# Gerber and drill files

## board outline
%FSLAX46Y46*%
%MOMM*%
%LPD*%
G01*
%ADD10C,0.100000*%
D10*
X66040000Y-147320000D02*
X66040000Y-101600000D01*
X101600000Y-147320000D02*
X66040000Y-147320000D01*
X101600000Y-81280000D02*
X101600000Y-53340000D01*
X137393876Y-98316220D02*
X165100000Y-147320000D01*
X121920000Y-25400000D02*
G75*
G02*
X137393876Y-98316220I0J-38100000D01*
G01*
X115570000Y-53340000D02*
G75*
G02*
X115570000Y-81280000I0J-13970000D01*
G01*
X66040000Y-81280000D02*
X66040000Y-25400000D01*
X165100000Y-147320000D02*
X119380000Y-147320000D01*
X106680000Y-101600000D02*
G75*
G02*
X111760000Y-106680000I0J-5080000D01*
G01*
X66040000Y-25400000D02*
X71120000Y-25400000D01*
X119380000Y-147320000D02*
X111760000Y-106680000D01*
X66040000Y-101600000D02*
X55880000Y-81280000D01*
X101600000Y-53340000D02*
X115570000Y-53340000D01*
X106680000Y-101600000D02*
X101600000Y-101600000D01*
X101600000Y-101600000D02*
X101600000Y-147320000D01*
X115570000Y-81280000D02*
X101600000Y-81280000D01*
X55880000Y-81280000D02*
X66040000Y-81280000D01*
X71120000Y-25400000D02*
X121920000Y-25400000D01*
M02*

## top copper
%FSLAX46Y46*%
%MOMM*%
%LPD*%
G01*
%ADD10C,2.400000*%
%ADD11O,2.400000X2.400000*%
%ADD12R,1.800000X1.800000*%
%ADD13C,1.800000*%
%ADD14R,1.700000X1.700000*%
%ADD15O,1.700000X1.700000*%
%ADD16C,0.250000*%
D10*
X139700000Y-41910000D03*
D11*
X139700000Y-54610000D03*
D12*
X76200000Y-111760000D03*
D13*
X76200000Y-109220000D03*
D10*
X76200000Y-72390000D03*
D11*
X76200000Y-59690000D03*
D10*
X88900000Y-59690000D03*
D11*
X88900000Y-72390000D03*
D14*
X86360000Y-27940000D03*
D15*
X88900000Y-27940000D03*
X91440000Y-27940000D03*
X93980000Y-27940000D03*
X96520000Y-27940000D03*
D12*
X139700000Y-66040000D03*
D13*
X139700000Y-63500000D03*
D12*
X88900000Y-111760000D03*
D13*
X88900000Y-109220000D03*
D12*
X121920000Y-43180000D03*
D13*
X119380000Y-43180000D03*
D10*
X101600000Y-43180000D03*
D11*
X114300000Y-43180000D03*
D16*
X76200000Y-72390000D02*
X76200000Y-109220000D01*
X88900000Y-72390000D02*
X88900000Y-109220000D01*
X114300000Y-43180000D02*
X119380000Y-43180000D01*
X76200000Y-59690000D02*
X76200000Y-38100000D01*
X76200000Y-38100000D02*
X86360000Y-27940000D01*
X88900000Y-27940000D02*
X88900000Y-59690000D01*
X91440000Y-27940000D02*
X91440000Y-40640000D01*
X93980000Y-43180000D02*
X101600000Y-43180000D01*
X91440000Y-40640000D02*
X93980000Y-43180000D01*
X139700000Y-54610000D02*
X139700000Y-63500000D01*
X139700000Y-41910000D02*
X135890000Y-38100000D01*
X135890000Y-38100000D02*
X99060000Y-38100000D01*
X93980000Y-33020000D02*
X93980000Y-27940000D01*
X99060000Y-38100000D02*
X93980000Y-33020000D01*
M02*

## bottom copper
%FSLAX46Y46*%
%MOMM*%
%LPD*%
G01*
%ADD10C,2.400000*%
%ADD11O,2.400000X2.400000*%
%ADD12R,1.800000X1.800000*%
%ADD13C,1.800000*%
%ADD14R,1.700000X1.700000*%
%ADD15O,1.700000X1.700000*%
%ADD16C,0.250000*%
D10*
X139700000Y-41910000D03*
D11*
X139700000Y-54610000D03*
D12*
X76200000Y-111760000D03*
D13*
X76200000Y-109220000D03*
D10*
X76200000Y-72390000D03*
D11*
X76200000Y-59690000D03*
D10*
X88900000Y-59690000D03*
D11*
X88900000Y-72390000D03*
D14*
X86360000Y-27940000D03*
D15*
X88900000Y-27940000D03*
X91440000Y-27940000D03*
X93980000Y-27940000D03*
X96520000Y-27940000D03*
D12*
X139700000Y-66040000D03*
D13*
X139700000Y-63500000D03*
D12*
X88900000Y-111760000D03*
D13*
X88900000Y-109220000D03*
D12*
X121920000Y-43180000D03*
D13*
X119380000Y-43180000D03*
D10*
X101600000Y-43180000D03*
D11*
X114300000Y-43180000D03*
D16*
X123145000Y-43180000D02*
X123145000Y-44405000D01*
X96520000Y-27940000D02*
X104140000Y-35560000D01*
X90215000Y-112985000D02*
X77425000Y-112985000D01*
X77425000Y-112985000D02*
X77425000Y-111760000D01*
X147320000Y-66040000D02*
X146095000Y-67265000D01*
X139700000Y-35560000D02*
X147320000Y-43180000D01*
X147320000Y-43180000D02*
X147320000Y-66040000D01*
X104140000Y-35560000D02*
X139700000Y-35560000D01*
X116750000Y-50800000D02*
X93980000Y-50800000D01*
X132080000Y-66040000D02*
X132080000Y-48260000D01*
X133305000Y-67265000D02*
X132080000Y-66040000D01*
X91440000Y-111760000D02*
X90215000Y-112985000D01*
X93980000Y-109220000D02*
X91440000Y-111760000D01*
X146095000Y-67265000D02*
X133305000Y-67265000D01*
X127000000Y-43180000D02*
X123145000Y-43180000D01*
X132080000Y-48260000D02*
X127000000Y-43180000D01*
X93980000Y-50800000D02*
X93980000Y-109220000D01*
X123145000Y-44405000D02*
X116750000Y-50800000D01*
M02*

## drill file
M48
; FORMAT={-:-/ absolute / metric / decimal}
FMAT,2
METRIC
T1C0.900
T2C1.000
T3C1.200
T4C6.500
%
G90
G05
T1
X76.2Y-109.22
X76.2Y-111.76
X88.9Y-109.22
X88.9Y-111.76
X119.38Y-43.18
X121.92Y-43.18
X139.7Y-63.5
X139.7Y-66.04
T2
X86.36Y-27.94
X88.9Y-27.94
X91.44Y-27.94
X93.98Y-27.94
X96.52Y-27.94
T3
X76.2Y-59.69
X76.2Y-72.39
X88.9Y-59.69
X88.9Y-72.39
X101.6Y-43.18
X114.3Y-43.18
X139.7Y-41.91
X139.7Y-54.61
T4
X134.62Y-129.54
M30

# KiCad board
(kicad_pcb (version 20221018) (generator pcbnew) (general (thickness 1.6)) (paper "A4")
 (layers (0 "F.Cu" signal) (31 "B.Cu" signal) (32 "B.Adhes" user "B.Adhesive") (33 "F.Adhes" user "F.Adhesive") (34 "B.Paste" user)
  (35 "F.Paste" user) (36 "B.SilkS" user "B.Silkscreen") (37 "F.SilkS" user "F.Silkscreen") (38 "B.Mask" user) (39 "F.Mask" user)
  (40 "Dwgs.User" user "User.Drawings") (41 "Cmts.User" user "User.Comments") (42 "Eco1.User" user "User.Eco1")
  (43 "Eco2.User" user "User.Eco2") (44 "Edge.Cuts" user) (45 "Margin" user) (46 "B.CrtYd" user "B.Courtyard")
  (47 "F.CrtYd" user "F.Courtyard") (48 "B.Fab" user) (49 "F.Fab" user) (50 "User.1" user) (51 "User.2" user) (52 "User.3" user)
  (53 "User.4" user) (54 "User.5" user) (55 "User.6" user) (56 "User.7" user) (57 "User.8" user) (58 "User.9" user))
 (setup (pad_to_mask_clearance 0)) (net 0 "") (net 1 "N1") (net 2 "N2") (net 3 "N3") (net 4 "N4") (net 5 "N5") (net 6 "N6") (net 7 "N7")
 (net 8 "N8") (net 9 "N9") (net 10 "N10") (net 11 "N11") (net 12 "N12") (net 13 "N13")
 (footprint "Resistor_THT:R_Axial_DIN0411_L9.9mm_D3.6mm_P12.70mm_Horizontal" (layer "F.Cu") (at 139.7 41.91 -90)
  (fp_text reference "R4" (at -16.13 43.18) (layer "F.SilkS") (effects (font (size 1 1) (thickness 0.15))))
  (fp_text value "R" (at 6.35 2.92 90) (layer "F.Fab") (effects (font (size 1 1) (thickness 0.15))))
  (pad "1" thru_hole circle (at 0 0 270) (size 2.4 2.4) (drill 1.2) (layers "*.Cu" "*.Mask") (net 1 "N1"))
  (pad "2" thru_hole oval (at 12.7 0 270) (size 2.4 2.4) (drill 1.2) (layers "*.Cu" "*.Mask") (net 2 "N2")))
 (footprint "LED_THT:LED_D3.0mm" (layer "F.Cu") (at 76.2 111.76 90)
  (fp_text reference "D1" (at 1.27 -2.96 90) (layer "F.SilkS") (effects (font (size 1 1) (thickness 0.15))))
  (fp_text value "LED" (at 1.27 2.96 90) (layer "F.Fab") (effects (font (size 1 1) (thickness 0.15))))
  (pad "1" thru_hole rect (at 0 0 90) (size 1.8 1.8) (drill 0.9) (layers "*.Cu" "*.Mask") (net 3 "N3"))
  (pad "2" thru_hole circle (at 2.54 0 90) (size 1.8 1.8) (drill 0.9) (layers "*.Cu" "*.Mask") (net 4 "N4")))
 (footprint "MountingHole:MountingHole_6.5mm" (layer "F.Cu") (at 134.62 129.54)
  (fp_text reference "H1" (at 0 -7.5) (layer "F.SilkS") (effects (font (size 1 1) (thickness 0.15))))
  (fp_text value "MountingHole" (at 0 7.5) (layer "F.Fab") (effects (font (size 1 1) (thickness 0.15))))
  (pad "" np_thru_hole circle (at 0 0) (size 6.5 6.5) (drill 6.5) (layers "*.Cu" "*.Mask")))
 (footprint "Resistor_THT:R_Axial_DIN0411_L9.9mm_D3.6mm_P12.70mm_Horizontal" (layer "F.Cu") (at 76.2 72.39 90)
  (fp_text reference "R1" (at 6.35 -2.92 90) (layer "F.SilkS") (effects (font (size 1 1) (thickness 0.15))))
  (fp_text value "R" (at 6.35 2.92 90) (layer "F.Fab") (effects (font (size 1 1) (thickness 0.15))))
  (pad "1" thru_hole circle (at 0 0 90) (size 2.4 2.4) (drill 1.2) (layers "*.Cu" "*.Mask") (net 4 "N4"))
  (pad "2" thru_hole oval (at 12.7 0 90) (size 2.4 2.4) (drill 1.2) (layers "*.Cu" "*.Mask") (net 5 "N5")))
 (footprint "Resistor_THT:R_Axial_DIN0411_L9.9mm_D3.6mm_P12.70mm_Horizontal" (layer "F.Cu") (at 88.9 59.69 -90)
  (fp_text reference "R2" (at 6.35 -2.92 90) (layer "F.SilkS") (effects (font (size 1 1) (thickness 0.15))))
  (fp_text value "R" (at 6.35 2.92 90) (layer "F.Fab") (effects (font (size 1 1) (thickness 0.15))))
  (pad "1" thru_hole circle (at 0 0 270) (size 2.4 2.4) (drill 1.2) (layers "*.Cu" "*.Mask") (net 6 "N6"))
  (pad "2" thru_hole oval (at 12.7 0 270) (size 2.4 2.4) (drill 1.2) (layers "*.Cu" "*.Mask") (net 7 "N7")))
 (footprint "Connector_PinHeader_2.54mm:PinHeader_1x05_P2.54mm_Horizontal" (layer "F.Cu") (at 86.36 27.94 90)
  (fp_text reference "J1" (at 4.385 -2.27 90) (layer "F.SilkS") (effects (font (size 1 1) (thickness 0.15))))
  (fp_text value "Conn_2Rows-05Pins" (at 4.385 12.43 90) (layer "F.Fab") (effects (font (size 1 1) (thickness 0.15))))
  (pad "1" thru_hole rect (at 0 0 90) (size 1.7 1.7) (drill 1) (layers "*.Cu" "*.Mask") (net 5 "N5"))
  (pad "2" thru_hole oval (at 0 2.54 90) (size 1.7 1.7) (drill 1) (layers "*.Cu" "*.Mask") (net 6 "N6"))
  (pad "3" thru_hole oval (at 0 5.08 90) (size 1.7 1.7) (drill 1) (layers "*.Cu" "*.Mask") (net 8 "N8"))
  (pad "4" thru_hole oval (at 0 7.62 90) (size 1.7 1.7) (drill 1) (layers "*.Cu" "*.Mask") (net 1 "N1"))
  (pad "5" thru_hole oval (at 0 10.16 90) (size 1.7 1.7) (drill 1) (layers "*.Cu" "*.Mask") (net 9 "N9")))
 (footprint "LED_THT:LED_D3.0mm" (layer "F.Cu") (at 139.7 66.04 90)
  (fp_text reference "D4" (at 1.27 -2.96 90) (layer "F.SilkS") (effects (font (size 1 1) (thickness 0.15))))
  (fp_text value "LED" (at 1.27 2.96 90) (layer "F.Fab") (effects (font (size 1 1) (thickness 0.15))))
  (pad "1" thru_hole rect (at 0 0 90) (size 1.8 1.8) (drill 0.9) (layers "*.Cu" "*.Mask") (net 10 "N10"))
  (pad "2" thru_hole circle (at 2.54 0 90) (size 1.8 1.8) (drill 0.9) (layers "*.Cu" "*.Mask") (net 2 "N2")))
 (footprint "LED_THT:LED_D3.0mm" (layer "F.Cu") (at 88.9 111.76 90)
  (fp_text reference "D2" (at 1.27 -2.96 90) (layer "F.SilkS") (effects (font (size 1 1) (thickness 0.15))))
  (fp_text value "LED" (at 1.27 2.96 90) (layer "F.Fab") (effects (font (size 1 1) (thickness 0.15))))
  (pad "1" thru_hole rect (at 0 0 90) (size 1.8 1.8) (drill 0.9) (layers "*.Cu" "*.Mask") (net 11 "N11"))
  (pad "2" thru_hole circle (at 2.54 0 90) (size 1.8 1.8) (drill 0.9) (layers "*.Cu" "*.Mask") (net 7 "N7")))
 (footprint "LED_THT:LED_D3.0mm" (layer "F.Cu") (at 121.92 43.18 180)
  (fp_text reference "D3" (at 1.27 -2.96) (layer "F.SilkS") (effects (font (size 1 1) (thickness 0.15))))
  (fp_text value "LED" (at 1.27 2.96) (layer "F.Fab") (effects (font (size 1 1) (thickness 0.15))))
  (pad "1" thru_hole rect (at 0 0 180) (size 1.8 1.8) (drill 0.9) (layers "*.Cu" "*.Mask") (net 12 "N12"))
  (pad "2" thru_hole circle (at 2.54 0 180) (size 1.8 1.8) (drill 0.9) (layers "*.Cu" "*.Mask") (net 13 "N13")))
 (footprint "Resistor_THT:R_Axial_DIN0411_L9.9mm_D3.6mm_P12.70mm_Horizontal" (layer "F.Cu") (at 101.6 43.18)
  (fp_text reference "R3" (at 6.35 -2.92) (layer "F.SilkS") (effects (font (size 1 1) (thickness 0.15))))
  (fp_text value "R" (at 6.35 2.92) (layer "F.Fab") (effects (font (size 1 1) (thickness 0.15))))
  (pad "1" thru_hole circle (at 0 0) (size 2.4 2.4) (drill 1.2) (layers "*.Cu" "*.Mask") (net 8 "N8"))
  (pad "2" thru_hole oval (at 12.7 0) (size 2.4 2.4) (drill 1.2) (layers "*.Cu" "*.Mask") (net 13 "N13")))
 (gr_line (start 66.04 147.32) (end 66.04 101.6) (stroke (width 0.1) (type default)) (layer "Edge.Cuts"))
 (gr_line (start 101.6 147.32) (end 66.04 147.32) (stroke (width 0.1) (type default)) (layer "Edge.Cuts"))
 (gr_line (start 101.6 81.28) (end 101.6 53.34) (stroke (width 0.1) (type default)) (layer "Edge.Cuts"))
 (gr_line (start 137.393876 98.31622) (end 165.1 147.32) (stroke (width 0.1) (type default)) (layer "Edge.Cuts"))
 (gr_arc (start 121.92 25.4) (mid 159.190015 55.590764) (end 137.393876 98.31622) (stroke (width 0.1) (type default)) (layer "Edge.Cuts"))
 (gr_arc (start 115.57 53.34) (mid 129.54 67.31) (end 115.57 81.28) (stroke (width 0.1) (type default)) (layer "Edge.Cuts"))
 (gr_line (start 66.04 81.28) (end 66.04 25.4) (stroke (width 0.1) (type default)) (layer "Edge.Cuts"))
 (gr_line (start 165.1 147.32) (end 119.38 147.32) (stroke (width 0.1) (type default)) (layer "Edge.Cuts"))
 (gr_arc (start 106.68 101.6) (mid 110.272102 103.087898) (end 111.76 106.68) (stroke (width 0.1) (type default)) (layer "Edge.Cuts"))
 (gr_line (start 66.04 25.4) (end 71.12 25.4) (stroke (width 0.1) (type default)) (layer "Edge.Cuts"))
 (gr_line (start 119.38 147.32) (end 111.76 106.68) (stroke (width 0.1) (type default)) (layer "Edge.Cuts"))
 (gr_line (start 66.04 101.6) (end 55.88 81.28) (stroke (width 0.1) (type default)) (layer "Edge.Cuts"))
 (gr_line (start 101.6 53.34) (end 115.57 53.34) (stroke (width 0.1) (type default)) (layer "Edge.Cuts"))
 (gr_line (start 106.68 101.6) (end 101.6 101.6) (stroke (width 0.1) (type default)) (layer "Edge.Cuts"))
 (gr_line (start 101.6 101.6) (end 101.6 147.32) (stroke (width 0.1) (type default)) (layer "Edge.Cuts"))
 (gr_line (start 115.57 81.28) (end 101.6 81.28) (stroke (width 0.1) (type default)) (layer "Edge.Cuts"))
 (gr_line (start 55.88 81.28) (end 66.04 81.28) (stroke (width 0.1) (type default)) (layer "Edge.Cuts"))
 (gr_line (start 71.12 25.4) (end 121.92 25.4) (stroke (width 0.1) (type default)) (layer "Edge.Cuts"))
 (segment (start 76.2 72.39) (end 76.2 109.22) (width 0.25) (layer "F.Cu") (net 4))
 (segment (start 88.9 72.39) (end 88.9 109.22) (width 0.25) (layer "F.Cu") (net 7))
 (segment (start 114.3 43.18) (end 119.38 43.18) (width 0.25) (layer "F.Cu") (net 13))
 (segment (start 76.2 59.69) (end 76.2 38.1) (width 0.25) (layer "F.Cu") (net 5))
 (segment (start 76.2 38.1) (end 86.36 27.94) (width 0.25) (layer "F.Cu") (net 5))
 (segment (start 88.9 27.94) (end 88.9 59.69) (width 0.25) (layer "F.Cu") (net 6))
 (segment (start 91.44 27.94) (end 91.44 40.64) (width 0.25) (layer "F.Cu") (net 8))
 (segment (start 93.98 43.18) (end 101.6 43.18) (width 0.25) (layer "F.Cu") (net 8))
 (segment (start 91.44 40.64) (end 93.98 43.18) (width 0.25) (layer "F.Cu") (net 8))
 (segment (start 139.7 54.61) (end 139.7 63.5) (width 0.25) (layer "F.Cu") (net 2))
 (segment (start 139.7 41.91) (end 135.89 38.1) (width 0.25) (layer "F.Cu") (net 1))
 (segment (start 135.89 38.1) (end 99.06 38.1) (width 0.25) (layer "F.Cu") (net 1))
 (segment (start 93.98 33.02) (end 93.98 27.94) (width 0.25) (layer "F.Cu") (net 1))
 (segment (start 99.06 38.1) (end 93.98 33.02) (width 0.25) (layer "F.Cu") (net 1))
 (segment (start 123.145 43.18) (end 123.145 44.405) (width 0.25) (layer "B.Cu") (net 9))
 (segment (start 96.52 27.94) (end 104.14 35.56) (width 0.25) (layer "B.Cu") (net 9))
 (segment (start 90.215 112.985) (end 77.425 112.985) (width 0.25) (layer "B.Cu") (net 9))
 (segment (start 77.425 112.985) (end 77.425 111.76) (width 0.25) (layer "B.Cu") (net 9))
 (segment (start 147.32 66.04) (end 146.095 67.265) (width 0.25) (layer "B.Cu") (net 9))
 (segment (start 139.7 35.56) (end 147.32 43.18) (width 0.25) (layer "B.Cu") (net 9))
 (segment (start 147.32 43.18) (end 147.32 66.04) (width 0.25) (layer "B.Cu") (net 9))
 (segment (start 104.14 35.56) (end 139.7 35.56) (width 0.25) (layer "B.Cu") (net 9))
 (segment (start 116.75 50.8) (end 93.98 50.8) (width 0.25) (layer "B.Cu") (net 9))
 (segment (start 132.08 66.04) (end 132.08 48.26) (width 0.25) (layer "B.Cu") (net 9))
 (segment (start 133.305 67.265) (end 132.08 66.04) (width 0.25) (layer "B.Cu") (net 9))
 (segment (start 91.44 111.76) (end 90.215 112.985) (width 0.25) (layer "B.Cu") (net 9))
 (segment (start 93.98 109.22) (end 91.44 111.76) (width 0.25) (layer "B.Cu") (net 9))
 (segment (start 146.095 67.265) (end 133.305 67.265) (width 0.25) (layer "B.Cu") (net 9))
 (segment (start 127 43.18) (end 123.145 43.18) (width 0.25) (layer "B.Cu") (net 9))
 (segment (start 132.08 48.26) (end 127 43.18) (width 0.25) (layer "B.Cu") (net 9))
 (segment (start 93.98 50.8) (end 93.98 109.22) (width 0.25) (layer "B.Cu") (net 9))
 (segment (start 123.145 44.405) (end 116.75 50.8) (width 0.25) (layer "B.Cu") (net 9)))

